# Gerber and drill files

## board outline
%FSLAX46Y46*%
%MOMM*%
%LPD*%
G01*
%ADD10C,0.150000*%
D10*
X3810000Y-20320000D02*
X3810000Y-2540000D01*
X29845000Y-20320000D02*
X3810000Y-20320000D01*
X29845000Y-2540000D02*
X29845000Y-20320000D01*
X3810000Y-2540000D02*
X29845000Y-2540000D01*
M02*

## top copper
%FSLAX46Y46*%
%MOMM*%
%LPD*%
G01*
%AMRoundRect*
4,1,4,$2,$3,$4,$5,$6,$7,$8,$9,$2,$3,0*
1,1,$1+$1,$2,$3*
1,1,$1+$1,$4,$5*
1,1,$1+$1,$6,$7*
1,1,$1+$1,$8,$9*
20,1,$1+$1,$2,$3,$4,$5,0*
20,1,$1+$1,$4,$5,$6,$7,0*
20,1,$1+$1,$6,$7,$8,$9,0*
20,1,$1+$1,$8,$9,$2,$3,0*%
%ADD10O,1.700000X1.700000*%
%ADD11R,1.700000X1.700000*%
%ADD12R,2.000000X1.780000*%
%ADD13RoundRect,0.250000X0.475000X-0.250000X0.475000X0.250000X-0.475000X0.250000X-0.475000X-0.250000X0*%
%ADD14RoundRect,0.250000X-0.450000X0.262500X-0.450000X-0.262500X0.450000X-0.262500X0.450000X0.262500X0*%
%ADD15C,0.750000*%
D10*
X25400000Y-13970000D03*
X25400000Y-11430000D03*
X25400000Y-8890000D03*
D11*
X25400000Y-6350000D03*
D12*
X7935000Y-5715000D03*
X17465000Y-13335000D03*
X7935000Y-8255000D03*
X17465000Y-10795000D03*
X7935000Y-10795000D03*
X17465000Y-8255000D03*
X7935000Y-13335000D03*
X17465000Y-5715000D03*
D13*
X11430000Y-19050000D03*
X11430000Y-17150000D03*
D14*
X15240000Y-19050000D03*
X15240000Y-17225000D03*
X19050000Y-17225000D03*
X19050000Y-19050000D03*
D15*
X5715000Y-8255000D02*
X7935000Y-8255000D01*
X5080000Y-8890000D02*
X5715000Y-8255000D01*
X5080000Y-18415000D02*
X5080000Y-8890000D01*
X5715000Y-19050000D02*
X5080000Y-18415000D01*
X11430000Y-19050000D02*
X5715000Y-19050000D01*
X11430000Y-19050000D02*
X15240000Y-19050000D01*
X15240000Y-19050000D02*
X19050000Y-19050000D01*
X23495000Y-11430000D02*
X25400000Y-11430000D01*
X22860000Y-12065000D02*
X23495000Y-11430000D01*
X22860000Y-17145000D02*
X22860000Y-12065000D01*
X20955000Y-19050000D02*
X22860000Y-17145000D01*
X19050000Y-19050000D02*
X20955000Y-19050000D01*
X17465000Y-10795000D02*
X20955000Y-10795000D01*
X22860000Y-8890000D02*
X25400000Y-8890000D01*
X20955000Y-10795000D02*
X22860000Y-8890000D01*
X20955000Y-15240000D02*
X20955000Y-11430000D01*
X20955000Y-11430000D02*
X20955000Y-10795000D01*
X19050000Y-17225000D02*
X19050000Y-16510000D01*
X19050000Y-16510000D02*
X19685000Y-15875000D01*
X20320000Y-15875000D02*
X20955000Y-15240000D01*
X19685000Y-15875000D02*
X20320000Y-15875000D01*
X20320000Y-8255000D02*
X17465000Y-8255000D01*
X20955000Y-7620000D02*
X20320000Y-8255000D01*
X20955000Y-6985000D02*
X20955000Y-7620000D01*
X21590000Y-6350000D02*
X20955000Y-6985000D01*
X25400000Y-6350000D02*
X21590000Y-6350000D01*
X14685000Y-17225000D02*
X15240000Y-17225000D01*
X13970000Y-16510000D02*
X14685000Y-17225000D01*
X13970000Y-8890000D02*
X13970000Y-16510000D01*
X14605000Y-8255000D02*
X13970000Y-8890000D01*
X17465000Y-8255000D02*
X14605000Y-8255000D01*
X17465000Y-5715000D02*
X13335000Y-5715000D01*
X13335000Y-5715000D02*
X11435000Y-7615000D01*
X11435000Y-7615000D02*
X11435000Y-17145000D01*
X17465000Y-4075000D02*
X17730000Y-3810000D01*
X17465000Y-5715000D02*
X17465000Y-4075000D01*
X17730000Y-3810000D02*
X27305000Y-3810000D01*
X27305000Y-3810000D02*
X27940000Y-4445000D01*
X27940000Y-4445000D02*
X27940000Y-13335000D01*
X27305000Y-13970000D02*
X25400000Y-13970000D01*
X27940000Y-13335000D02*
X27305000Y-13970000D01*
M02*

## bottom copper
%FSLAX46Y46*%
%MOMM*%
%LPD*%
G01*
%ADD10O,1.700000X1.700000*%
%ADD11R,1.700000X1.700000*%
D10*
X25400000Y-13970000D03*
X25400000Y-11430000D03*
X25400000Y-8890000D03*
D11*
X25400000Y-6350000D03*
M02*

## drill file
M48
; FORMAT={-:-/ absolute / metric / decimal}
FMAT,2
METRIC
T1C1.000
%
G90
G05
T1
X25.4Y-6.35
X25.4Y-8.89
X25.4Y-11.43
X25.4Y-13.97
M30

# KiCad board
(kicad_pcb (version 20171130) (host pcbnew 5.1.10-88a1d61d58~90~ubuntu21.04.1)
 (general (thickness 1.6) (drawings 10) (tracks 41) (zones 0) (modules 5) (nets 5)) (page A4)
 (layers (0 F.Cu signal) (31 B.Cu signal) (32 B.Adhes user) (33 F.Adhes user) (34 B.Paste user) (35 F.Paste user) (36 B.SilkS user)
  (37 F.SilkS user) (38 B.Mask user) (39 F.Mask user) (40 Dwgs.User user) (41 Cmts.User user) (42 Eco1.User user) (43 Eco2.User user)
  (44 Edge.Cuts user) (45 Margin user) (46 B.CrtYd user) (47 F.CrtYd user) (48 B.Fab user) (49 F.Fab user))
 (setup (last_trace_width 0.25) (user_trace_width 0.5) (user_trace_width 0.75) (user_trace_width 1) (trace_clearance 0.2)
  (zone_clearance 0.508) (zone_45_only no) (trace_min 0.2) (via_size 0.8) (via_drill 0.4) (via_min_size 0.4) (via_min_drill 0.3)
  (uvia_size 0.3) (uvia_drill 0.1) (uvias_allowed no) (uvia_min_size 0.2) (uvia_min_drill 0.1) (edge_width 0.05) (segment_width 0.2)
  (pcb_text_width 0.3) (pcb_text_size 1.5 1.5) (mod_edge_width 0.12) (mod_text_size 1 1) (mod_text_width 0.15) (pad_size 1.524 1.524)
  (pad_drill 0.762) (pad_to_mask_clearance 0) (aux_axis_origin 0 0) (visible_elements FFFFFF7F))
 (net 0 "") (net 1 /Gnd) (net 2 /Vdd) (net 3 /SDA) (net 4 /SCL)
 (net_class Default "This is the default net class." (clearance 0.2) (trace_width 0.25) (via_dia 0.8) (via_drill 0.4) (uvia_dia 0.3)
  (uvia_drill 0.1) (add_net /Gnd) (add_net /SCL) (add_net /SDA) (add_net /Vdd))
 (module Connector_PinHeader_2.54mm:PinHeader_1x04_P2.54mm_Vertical (layer F.Cu) (at 25.4 6.35)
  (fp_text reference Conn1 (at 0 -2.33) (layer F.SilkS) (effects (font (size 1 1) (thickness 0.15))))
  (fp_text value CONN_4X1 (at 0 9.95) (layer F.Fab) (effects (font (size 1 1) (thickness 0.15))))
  (pad 4 thru_hole oval (at 0 7.62) (size 1.7 1.7) (drill 1) (layers *.Cu *.Mask) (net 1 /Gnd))
  (pad 3 thru_hole oval (at 0 5.08) (size 1.7 1.7) (drill 1) (layers *.Cu *.Mask) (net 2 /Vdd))
  (pad 2 thru_hole oval (at 0 2.54) (size 1.7 1.7) (drill 1) (layers *.Cu *.Mask) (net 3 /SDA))
  (pad 1 thru_hole rect (at 0 0) (size 1.7 1.7) (drill 1) (layers *.Cu *.Mask) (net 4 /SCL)))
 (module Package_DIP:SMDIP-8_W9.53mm (layer F.Cu) (at 12.7 9.525)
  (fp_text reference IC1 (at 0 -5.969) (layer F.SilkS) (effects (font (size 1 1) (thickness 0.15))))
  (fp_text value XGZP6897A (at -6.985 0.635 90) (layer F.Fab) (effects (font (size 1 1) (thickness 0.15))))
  (pad 1 smd rect (at -4.765 -3.81) (size 2 1.78) (layers F.Cu F.Paste F.Mask))
  (pad 5 smd rect (at 4.765 3.81) (size 2 1.78) (layers F.Cu F.Paste F.Mask))
  (pad 2 smd rect (at -4.765 -1.27) (size 2 1.78) (layers F.Cu F.Paste F.Mask) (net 2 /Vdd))
  (pad 6 smd rect (at 4.765 1.27) (size 2 1.78) (layers F.Cu F.Paste F.Mask) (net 3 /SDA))
  (pad 3 smd rect (at -4.765 1.27) (size 2 1.78) (layers F.Cu F.Paste F.Mask))
  (pad 7 smd rect (at 4.765 -1.27) (size 2 1.78) (layers F.Cu F.Paste F.Mask) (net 4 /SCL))
  (pad 4 smd rect (at -4.765 3.81) (size 2 1.78) (layers F.Cu F.Paste F.Mask))
  (pad 8 smd rect (at 4.765 -3.81) (size 2 1.78) (layers F.Cu F.Paste F.Mask) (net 1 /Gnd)))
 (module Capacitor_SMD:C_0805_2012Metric (layer F.Cu) (at 11.43 18.1 90)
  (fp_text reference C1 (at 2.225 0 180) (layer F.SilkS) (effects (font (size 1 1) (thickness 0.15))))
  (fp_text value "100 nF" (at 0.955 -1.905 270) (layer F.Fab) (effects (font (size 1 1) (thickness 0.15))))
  (pad 1 smd roundrect (at -0.95 0 90) (size 1 1.45) (layers F.Cu F.Paste F.Mask) (roundrect_rratio 0.25) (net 2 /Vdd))
  (pad 2 smd roundrect (at 0.95 0 90) (size 1 1.45) (layers F.Cu F.Paste F.Mask) (roundrect_rratio 0.25) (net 1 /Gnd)))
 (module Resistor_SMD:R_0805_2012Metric (layer F.Cu) (at 15.24 18.1375 270)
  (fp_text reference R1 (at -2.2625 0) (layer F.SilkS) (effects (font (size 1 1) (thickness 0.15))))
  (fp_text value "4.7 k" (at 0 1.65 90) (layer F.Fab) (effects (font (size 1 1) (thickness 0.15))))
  (pad 2 smd roundrect (at 0.9125 0 270) (size 1.025 1.4) (layers F.Cu F.Paste F.Mask) (roundrect_rratio 0.243902) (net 2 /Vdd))
  (pad 1 smd roundrect (at -0.9125 0 270) (size 1.025 1.4) (layers F.Cu F.Paste F.Mask) (roundrect_rratio 0.243902) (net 4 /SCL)))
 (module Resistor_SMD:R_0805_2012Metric (layer F.Cu) (at 19.05 18.1375 270)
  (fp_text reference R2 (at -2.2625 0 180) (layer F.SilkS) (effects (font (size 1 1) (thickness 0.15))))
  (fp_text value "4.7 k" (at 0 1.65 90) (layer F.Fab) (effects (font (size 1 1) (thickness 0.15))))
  (pad 1 smd roundrect (at -0.9125 0 270) (size 1.025 1.4) (layers F.Cu F.Paste F.Mask) (roundrect_rratio 0.243902) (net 3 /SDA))
  (pad 2 smd roundrect (at 0.9125 0 270) (size 1.025 1.4) (layers F.Cu F.Paste F.Mask) (roundrect_rratio 0.243902) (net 2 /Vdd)))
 (gr_line (start 3.81 20.32) (end 3.81 2.54) (layer Edge.Cuts) (width 0.15))
 (gr_line (start 29.845 20.32) (end 3.81 20.32) (layer Edge.Cuts) (width 0.15))
 (gr_line (start 29.845 2.54) (end 29.845 20.32) (layer Edge.Cuts) (width 0.15))
 (gr_line (start 3.81 2.54) (end 29.845 2.54) (layer Edge.Cuts) (width 0.15))
 (segment (start 5.715 8.255) (end 7.935 8.255) (width 0.75) (layer F.Cu) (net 2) (status 20))
 (segment (start 5.08 8.89) (end 5.715 8.255) (width 0.75) (layer F.Cu) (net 2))
 (segment (start 5.08 18.415) (end 5.08 8.89) (width 0.75) (layer F.Cu) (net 2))
 (segment (start 5.715 19.05) (end 5.08 18.415) (width 0.75) (layer F.Cu) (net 2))
 (segment (start 11.43 19.05) (end 5.715 19.05) (width 0.75) (layer F.Cu) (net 2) (status 10))
 (segment (start 11.43 19.05) (end 15.24 19.05) (width 0.75) (layer F.Cu) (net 2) (status 30))
 (segment (start 15.24 19.05) (end 19.05 19.05) (width 0.75) (layer F.Cu) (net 2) (status 30))
 (segment (start 23.495 11.43) (end 25.4 11.43) (width 0.75) (layer F.Cu) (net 2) (status 20))
 (segment (start 22.86 12.065) (end 23.495 11.43) (width 0.75) (layer F.Cu) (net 2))
 (segment (start 22.86 17.145) (end 22.86 12.065) (width 0.75) (layer F.Cu) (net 2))
 (segment (start 20.955 19.05) (end 22.86 17.145) (width 0.75) (layer F.Cu) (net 2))
 (segment (start 19.05 19.05) (end 20.955 19.05) (width 0.75) (layer F.Cu) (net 2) (status 10))
 (segment (start 17.465 10.795) (end 20.955 10.795) (width 0.75) (layer F.Cu) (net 3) (status 10))
 (segment (start 22.86 8.89) (end 25.4 8.89) (width 0.75) (layer F.Cu) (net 3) (status 20))
 (segment (start 20.955 10.795) (end 22.86 8.89) (width 0.75) (layer F.Cu) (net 3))
 (segment (start 20.955 15.24) (end 20.955 11.43) (width 0.75) (layer F.Cu) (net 3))
 (segment (start 20.955 11.43) (end 20.955 10.795) (width 0.75) (layer F.Cu) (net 3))
 (segment (start 19.05 17.225) (end 19.05 16.51) (width 0.75) (layer F.Cu) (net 3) (status 10))
 (segment (start 19.05 16.51) (end 19.685 15.875) (width 0.75) (layer F.Cu) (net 3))
 (segment (start 20.32 15.875) (end 20.955 15.24) (width 0.75) (layer F.Cu) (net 3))
 (segment (start 19.685 15.875) (end 20.32 15.875) (width 0.75) (layer F.Cu) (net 3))
 (segment (start 20.32 8.255) (end 17.465 8.255) (width 0.75) (layer F.Cu) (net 4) (status 20))
 (segment (start 20.955 7.62) (end 20.32 8.255) (width 0.75) (layer F.Cu) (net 4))
 (segment (start 20.955 6.985) (end 20.955 7.62) (width 0.75) (layer F.Cu) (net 4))
 (segment (start 21.59 6.35) (end 20.955 6.985) (width 0.75) (layer F.Cu) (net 4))
 (segment (start 25.4 6.35) (end 21.59 6.35) (width 0.75) (layer F.Cu) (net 4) (status 10))
 (segment (start 14.685 17.225) (end 15.24 17.225) (width 0.75) (layer F.Cu) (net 4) (status 30))
 (segment (start 13.97 16.51) (end 14.685 17.225) (width 0.75) (layer F.Cu) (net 4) (status 20))
 (segment (start 13.97 8.89) (end 13.97 16.51) (width 0.75) (layer F.Cu) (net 4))
 (segment (start 14.605 8.255) (end 13.97 8.89) (width 0.75) (layer F.Cu) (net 4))
 (segment (start 17.465 8.255) (end 14.605 8.255) (width 0.75) (layer F.Cu) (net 4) (status 10))
 (segment (start 17.465 5.715) (end 13.335 5.715) (width 0.75) (layer F.Cu) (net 1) (status 10))
 (segment (start 13.335 5.715) (end 11.435 7.615) (width 0.75) (layer F.Cu) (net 1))
 (segment (start 11.435 7.615) (end 11.435 17.145) (width 0.75) (layer F.Cu) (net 1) (status 20))
 (segment (start 17.465 4.075) (end 17.73 3.81) (width 0.75) (layer F.Cu) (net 1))
 (segment (start 17.465 5.715) (end 17.465 4.075) (width 0.75) (layer F.Cu) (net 1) (status 10))
 (segment (start 17.73 3.81) (end 27.305 3.81) (width 0.75) (layer F.Cu) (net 1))
 (segment (start 27.305 3.81) (end 27.94 4.445) (width 0.75) (layer F.Cu) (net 1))
 (segment (start 27.94 4.445) (end 27.94 13.335) (width 0.75) (layer F.Cu) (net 1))
 (segment (start 27.305 13.97) (end 25.4 13.97) (width 0.75) (layer F.Cu) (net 1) (status 20))
 (segment (start 27.94 13.335) (end 27.305 13.97) (width 0.75) (layer F.Cu) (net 1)))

